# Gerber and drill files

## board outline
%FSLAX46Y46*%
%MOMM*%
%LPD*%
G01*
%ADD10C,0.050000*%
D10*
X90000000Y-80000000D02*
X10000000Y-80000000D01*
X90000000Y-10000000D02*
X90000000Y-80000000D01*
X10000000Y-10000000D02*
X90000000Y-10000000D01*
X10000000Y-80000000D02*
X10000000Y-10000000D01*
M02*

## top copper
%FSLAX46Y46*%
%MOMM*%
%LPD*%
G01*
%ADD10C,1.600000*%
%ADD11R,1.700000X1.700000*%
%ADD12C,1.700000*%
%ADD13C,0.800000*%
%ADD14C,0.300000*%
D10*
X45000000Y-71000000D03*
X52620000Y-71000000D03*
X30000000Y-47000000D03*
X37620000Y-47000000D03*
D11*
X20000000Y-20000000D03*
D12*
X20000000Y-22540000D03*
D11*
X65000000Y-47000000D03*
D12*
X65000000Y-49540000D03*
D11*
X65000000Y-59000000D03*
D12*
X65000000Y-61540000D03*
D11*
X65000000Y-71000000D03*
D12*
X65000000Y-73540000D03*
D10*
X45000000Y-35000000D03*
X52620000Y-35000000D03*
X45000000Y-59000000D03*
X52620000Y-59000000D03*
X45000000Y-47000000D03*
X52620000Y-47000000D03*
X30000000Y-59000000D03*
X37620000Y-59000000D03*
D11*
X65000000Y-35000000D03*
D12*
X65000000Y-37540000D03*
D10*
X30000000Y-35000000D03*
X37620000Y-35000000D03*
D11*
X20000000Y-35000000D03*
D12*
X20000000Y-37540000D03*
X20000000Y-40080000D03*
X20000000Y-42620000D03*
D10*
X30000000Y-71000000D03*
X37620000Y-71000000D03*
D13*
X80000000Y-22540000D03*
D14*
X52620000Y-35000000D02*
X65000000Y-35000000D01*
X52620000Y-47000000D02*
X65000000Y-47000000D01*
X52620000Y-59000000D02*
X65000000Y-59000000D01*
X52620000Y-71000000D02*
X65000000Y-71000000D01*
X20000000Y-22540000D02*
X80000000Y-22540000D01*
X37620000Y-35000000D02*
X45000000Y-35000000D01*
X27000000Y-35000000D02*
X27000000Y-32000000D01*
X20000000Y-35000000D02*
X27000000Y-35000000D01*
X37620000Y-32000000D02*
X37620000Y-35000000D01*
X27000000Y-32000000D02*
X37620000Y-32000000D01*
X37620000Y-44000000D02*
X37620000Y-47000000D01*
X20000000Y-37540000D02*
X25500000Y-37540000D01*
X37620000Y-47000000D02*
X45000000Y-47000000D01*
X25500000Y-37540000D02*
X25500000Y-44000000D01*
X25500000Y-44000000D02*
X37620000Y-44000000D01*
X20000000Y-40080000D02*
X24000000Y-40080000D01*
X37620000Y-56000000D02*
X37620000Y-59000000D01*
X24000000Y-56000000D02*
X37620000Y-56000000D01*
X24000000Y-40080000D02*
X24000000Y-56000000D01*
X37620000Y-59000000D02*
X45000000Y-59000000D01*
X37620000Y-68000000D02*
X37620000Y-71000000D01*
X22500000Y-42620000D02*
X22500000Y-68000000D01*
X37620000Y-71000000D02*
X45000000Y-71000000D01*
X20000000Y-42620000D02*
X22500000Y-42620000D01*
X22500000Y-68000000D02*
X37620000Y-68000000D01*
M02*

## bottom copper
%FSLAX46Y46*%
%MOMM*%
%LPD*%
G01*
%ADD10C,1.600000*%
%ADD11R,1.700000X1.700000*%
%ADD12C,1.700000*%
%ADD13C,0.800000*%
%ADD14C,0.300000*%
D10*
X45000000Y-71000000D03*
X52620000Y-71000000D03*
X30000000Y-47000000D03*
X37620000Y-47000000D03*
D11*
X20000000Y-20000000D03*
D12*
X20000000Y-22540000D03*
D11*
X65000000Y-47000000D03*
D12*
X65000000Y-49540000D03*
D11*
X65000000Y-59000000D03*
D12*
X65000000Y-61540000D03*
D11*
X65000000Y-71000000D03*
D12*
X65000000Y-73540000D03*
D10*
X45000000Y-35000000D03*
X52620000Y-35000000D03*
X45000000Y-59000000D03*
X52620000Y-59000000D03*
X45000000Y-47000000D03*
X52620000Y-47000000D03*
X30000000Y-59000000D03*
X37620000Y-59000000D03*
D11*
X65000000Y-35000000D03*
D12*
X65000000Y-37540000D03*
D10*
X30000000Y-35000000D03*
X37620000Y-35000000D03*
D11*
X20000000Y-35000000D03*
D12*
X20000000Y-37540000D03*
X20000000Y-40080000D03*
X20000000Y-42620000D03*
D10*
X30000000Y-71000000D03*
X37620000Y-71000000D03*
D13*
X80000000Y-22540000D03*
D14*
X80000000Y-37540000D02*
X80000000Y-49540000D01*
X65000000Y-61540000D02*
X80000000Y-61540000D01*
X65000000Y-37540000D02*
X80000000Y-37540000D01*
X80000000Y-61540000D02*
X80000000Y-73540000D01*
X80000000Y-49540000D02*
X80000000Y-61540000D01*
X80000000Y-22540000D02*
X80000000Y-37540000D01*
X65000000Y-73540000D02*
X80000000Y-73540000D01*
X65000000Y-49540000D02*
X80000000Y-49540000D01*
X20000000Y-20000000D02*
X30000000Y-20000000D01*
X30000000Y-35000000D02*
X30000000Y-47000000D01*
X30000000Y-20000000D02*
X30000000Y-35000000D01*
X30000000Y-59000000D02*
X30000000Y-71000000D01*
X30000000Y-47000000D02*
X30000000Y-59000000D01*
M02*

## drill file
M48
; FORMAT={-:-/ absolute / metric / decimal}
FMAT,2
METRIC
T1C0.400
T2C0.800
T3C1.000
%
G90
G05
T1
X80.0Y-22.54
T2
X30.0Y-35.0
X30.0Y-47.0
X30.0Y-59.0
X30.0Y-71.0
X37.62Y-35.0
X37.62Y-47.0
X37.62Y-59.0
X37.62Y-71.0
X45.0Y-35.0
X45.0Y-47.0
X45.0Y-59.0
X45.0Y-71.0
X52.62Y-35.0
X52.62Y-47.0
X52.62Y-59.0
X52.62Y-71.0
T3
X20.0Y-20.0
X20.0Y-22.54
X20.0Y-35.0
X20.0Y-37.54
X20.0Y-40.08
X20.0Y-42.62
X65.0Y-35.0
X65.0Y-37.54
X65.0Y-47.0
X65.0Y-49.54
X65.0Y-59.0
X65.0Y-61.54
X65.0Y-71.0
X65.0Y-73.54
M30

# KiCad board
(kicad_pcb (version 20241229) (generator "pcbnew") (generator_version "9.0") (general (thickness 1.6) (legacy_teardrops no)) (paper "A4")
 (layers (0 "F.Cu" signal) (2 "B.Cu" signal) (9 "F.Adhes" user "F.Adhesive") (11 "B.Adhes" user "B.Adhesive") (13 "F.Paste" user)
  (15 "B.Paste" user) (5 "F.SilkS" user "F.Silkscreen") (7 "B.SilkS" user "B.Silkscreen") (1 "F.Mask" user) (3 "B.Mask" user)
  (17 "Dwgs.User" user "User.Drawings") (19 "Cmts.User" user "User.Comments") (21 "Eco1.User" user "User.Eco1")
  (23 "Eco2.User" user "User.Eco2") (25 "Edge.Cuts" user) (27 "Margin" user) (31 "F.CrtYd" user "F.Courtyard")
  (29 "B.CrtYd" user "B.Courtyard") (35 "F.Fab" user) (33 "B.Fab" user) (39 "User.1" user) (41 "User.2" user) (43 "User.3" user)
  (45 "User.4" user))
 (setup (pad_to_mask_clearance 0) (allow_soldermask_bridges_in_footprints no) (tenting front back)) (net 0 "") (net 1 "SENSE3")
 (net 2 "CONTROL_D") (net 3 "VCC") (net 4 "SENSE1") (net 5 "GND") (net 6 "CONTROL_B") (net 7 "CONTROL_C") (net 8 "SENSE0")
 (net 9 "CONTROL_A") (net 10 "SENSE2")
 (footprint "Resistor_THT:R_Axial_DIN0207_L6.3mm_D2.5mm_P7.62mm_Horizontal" (layer "F.Cu") (at 45 71)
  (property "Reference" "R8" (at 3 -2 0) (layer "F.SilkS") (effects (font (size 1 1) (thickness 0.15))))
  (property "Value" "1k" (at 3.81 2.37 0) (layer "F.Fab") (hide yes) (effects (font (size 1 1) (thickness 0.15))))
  (pad "1" thru_hole circle (at 0 0) (size 1.6 1.6) (drill 0.8) (layers "*.Cu" "*.Mask") (remove_unused_layers no) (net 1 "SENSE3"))
  (pad "2" thru_hole circle (at 7.62 0) (size 1.6 1.6) (drill 0.8) (layers "*.Cu" "*.Mask") (remove_unused_layers no) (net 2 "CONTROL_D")))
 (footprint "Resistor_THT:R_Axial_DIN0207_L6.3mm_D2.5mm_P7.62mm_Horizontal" (layer "F.Cu") (at 30 47)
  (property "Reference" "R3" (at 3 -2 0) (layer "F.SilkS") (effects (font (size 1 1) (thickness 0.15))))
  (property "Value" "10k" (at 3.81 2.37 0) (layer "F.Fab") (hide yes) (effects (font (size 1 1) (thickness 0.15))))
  (pad "1" thru_hole circle (at 0 0) (size 1.6 1.6) (drill 0.8) (layers "*.Cu" "*.Mask") (remove_unused_layers no) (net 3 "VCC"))
  (pad "2" thru_hole circle (at 7.62 0) (size 1.6 1.6) (drill 0.8) (layers "*.Cu" "*.Mask") (remove_unused_layers no) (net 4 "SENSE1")))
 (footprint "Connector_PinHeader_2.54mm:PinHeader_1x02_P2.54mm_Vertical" (layer "F.Cu") (at 20 20)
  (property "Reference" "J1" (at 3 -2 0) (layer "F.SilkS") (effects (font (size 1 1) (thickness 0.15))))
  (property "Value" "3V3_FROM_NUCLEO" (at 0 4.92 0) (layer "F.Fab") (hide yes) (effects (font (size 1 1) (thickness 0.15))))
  (pad "1" thru_hole rect (at 0 0) (size 1.7 1.7) (drill 1) (layers "*.Cu" "*.Mask") (remove_unused_layers no) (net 3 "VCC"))
  (pad "2" thru_hole circle (at 0 2.54) (size 1.7 1.7) (drill 1) (layers "*.Cu" "*.Mask") (remove_unused_layers no) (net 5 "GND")))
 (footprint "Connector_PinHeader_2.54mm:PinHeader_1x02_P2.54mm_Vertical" (layer "F.Cu") (at 65 47)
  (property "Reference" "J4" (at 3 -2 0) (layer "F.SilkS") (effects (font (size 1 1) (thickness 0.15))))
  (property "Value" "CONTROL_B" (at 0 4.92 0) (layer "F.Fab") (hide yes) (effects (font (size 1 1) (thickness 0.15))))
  (pad "1" thru_hole rect (at 0 0) (size 1.7 1.7) (drill 1) (layers "*.Cu" "*.Mask") (remove_unused_layers no) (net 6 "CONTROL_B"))
  (pad "2" thru_hole circle (at 0 2.54) (size 1.7 1.7) (drill 1) (layers "*.Cu" "*.Mask") (remove_unused_layers no) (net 5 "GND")))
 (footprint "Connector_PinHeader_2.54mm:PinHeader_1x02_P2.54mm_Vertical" (layer "F.Cu") (at 65 59)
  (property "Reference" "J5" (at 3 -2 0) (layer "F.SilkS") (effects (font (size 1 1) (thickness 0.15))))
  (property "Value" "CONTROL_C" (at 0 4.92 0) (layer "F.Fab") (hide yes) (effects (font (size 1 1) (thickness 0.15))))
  (pad "1" thru_hole rect (at 0 0) (size 1.7 1.7) (drill 1) (layers "*.Cu" "*.Mask") (remove_unused_layers no) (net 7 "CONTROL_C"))
  (pad "2" thru_hole circle (at 0 2.54) (size 1.7 1.7) (drill 1) (layers "*.Cu" "*.Mask") (remove_unused_layers no) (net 5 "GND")))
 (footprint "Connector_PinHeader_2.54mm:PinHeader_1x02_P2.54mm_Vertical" (layer "F.Cu") (at 65 71)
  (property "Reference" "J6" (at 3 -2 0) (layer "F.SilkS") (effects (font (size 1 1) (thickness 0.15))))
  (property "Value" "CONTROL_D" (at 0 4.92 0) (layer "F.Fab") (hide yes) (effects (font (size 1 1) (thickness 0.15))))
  (pad "1" thru_hole rect (at 0 0) (size 1.7 1.7) (drill 1) (layers "*.Cu" "*.Mask") (remove_unused_layers no) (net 2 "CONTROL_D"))
  (pad "2" thru_hole circle (at 0 2.54) (size 1.7 1.7) (drill 1) (layers "*.Cu" "*.Mask") (remove_unused_layers no) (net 5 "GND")))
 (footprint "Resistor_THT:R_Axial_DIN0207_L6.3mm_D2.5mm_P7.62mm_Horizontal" (layer "F.Cu") (at 45 35)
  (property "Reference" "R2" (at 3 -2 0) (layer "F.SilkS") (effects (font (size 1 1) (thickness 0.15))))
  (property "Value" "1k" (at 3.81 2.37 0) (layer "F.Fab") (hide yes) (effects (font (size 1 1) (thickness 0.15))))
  (pad "1" thru_hole circle (at 0 0) (size 1.6 1.6) (drill 0.8) (layers "*.Cu" "*.Mask") (remove_unused_layers no) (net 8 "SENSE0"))
  (pad "2" thru_hole circle (at 7.62 0) (size 1.6 1.6) (drill 0.8) (layers "*.Cu" "*.Mask") (remove_unused_layers no) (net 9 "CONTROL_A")))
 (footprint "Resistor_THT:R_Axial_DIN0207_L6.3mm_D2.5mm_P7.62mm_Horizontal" (layer "F.Cu") (at 45 59)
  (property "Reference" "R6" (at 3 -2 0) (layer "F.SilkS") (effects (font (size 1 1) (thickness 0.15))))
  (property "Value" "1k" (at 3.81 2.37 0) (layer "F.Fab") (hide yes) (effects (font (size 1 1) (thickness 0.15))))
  (pad "1" thru_hole circle (at 0 0) (size 1.6 1.6) (drill 0.8) (layers "*.Cu" "*.Mask") (remove_unused_layers no) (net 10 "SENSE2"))
  (pad "2" thru_hole circle (at 7.62 0) (size 1.6 1.6) (drill 0.8) (layers "*.Cu" "*.Mask") (remove_unused_layers no) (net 7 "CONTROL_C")))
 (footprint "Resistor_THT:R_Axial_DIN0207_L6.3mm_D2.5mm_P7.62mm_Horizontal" (layer "F.Cu") (at 45 47)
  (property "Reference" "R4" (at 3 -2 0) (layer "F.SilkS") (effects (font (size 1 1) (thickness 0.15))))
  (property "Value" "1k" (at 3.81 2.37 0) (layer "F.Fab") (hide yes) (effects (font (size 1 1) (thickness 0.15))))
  (pad "1" thru_hole circle (at 0 0) (size 1.6 1.6) (drill 0.8) (layers "*.Cu" "*.Mask") (remove_unused_layers no) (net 4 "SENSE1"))
  (pad "2" thru_hole circle (at 7.62 0) (size 1.6 1.6) (drill 0.8) (layers "*.Cu" "*.Mask") (remove_unused_layers no) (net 6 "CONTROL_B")))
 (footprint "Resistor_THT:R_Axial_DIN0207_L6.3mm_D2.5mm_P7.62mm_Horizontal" (layer "F.Cu") (at 30 59)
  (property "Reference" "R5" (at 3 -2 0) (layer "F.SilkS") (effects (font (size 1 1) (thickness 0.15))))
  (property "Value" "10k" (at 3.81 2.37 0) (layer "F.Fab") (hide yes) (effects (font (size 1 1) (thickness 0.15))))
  (pad "1" thru_hole circle (at 0 0) (size 1.6 1.6) (drill 0.8) (layers "*.Cu" "*.Mask") (remove_unused_layers no) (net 3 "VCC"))
  (pad "2" thru_hole circle (at 7.62 0) (size 1.6 1.6) (drill 0.8) (layers "*.Cu" "*.Mask") (remove_unused_layers no) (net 10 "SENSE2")))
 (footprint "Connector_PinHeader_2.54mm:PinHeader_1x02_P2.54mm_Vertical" (layer "F.Cu") (at 65 35)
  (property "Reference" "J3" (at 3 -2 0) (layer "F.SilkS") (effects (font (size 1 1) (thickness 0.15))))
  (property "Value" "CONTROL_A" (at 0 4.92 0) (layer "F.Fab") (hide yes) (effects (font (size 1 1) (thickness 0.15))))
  (pad "1" thru_hole rect (at 0 0) (size 1.7 1.7) (drill 1) (layers "*.Cu" "*.Mask") (remove_unused_layers no) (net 9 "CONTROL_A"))
  (pad "2" thru_hole circle (at 0 2.54) (size 1.7 1.7) (drill 1) (layers "*.Cu" "*.Mask") (remove_unused_layers no) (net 5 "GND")))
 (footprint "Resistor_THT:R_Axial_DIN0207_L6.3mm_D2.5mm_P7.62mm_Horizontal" (layer "F.Cu") (at 30 35)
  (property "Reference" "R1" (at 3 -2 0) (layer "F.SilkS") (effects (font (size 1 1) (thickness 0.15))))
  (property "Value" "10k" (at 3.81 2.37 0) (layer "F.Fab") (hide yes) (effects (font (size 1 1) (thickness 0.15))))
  (pad "1" thru_hole circle (at 0 0) (size 1.6 1.6) (drill 0.8) (layers "*.Cu" "*.Mask") (remove_unused_layers no) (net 3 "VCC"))
  (pad "2" thru_hole circle (at 7.62 0) (size 1.6 1.6) (drill 0.8) (layers "*.Cu" "*.Mask") (remove_unused_layers no) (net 8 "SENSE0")))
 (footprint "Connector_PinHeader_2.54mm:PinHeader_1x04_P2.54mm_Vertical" (layer "F.Cu") (at 20 35)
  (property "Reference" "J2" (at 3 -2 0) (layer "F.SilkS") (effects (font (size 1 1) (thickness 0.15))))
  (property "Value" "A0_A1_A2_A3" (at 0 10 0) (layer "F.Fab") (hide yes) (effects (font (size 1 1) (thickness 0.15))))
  (pad "1" thru_hole rect (at 0 0) (size 1.7 1.7) (drill 1) (layers "*.Cu" "*.Mask") (remove_unused_layers no) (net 8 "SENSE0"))
  (pad "2" thru_hole circle (at 0 2.54) (size 1.7 1.7) (drill 1) (layers "*.Cu" "*.Mask") (remove_unused_layers no) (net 4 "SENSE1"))
  (pad "3" thru_hole circle (at 0 5.08) (size 1.7 1.7) (drill 1) (layers "*.Cu" "*.Mask") (remove_unused_layers no) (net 10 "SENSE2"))
  (pad "4" thru_hole circle (at 0 7.62) (size 1.7 1.7) (drill 1) (layers "*.Cu" "*.Mask") (remove_unused_layers no) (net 1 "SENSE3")))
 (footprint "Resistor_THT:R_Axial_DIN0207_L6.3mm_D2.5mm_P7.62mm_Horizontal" (layer "F.Cu") (at 30 71)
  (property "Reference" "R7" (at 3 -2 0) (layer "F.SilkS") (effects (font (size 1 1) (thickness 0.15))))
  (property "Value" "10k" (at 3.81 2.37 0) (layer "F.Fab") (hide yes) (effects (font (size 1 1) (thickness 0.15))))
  (pad "1" thru_hole circle (at 0 0) (size 1.6 1.6) (drill 0.8) (layers "*.Cu" "*.Mask") (remove_unused_layers no) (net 3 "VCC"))
  (pad "2" thru_hole circle (at 7.62 0) (size 1.6 1.6) (drill 0.8) (layers "*.Cu" "*.Mask") (remove_unused_layers no) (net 1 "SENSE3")))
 (gr_line (start 90 80) (end 10 80) (stroke (width 0.05) (type default)) (layer "Edge.Cuts"))
 (gr_line (start 90 10) (end 90 80) (stroke (width 0.05) (type default)) (layer "Edge.Cuts"))
 (gr_line (start 10 10) (end 90 10) (stroke (width 0.05) (type default)) (layer "Edge.Cuts"))
 (gr_line (start 10 80) (end 10 10) (stroke (width 0.05) (type default)) (layer "Edge.Cuts"))
 (segment (start 52.62 35) (end 65 35) (width 0.3) (layer "F.Cu") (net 9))
 (segment (start 52.62 47) (end 65 47) (width 0.3) (layer "F.Cu") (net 6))
 (segment (start 52.62 59) (end 65 59) (width 0.3) (layer "F.Cu") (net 7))
 (segment (start 52.62 71) (end 65 71) (width 0.3) (layer "F.Cu") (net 2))
 (segment (start 20 22.54) (end 80 22.54) (width 0.3) (layer "F.Cu") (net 5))
 (via (at 80 22.54) (size 0.8) (drill 0.4) (layers "F.Cu" "B.Cu") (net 5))
 (segment (start 80 37.54) (end 80 49.54) (width 0.3) (layer "B.Cu") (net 5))
 (segment (start 65 61.54) (end 80 61.54) (width 0.3) (layer "B.Cu") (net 5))
 (segment (start 65 37.54) (end 80 37.54) (width 0.3) (layer "B.Cu") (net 5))
 (segment (start 80 61.54) (end 80 73.54) (width 0.3) (layer "B.Cu") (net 5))
 (segment (start 80 49.54) (end 80 61.54) (width 0.3) (layer "B.Cu") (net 5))
 (segment (start 80 22.54) (end 80 37.54) (width 0.3) (layer "B.Cu") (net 5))
 (segment (start 65 73.54) (end 80 73.54) (width 0.3) (layer "B.Cu") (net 5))
 (segment (start 65 49.54) (end 80 49.54) (width 0.3) (layer "B.Cu") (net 5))
 (segment (start 37.62 35) (end 45 35) (width 0.3) (layer "F.Cu") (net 8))
 (segment (start 27 35) (end 27 32) (width 0.3) (layer "F.Cu") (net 8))
 (segment (start 20 35) (end 27 35) (width 0.3) (layer "F.Cu") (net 8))
 (segment (start 37.62 32) (end 37.62 35) (width 0.3) (layer "F.Cu") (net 8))
 (segment (start 27 32) (end 37.62 32) (width 0.3) (layer "F.Cu") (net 8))
 (segment (start 37.62 44) (end 37.62 47) (width 0.3) (layer "F.Cu") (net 4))
 (segment (start 20 37.54) (end 25.5 37.54) (width 0.3) (layer "F.Cu") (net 4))
 (segment (start 37.62 47) (end 45 47) (width 0.3) (layer "F.Cu") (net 4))
 (segment (start 25.5 37.54) (end 25.5 44) (width 0.3) (layer "F.Cu") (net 4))
 (segment (start 25.5 44) (end 37.62 44) (width 0.3) (layer "F.Cu") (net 4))
 (segment (start 20 40.08) (end 24 40.08) (width 0.3) (layer "F.Cu") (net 10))
 (segment (start 37.62 56) (end 37.62 59) (width 0.3) (layer "F.Cu") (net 10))
 (segment (start 24 56) (end 37.62 56) (width 0.3) (layer "F.Cu") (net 10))
 (segment (start 24 40.08) (end 24 56) (width 0.3) (layer "F.Cu") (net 10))
 (segment (start 37.62 59) (end 45 59) (width 0.3) (layer "F.Cu") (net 10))
 (segment (start 37.62 68) (end 37.62 71) (width 0.3) (layer "F.Cu") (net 1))
 (segment (start 22.5 42.62) (end 22.5 68) (width 0.3) (layer "F.Cu") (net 1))
 (segment (start 37.62 71) (end 45 71) (width 0.3) (layer "F.Cu") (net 1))
 (segment (start 20 42.62) (end 22.5 42.62) (width 0.3) (layer "F.Cu") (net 1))
 (segment (start 22.5 68) (end 37.62 68) (width 0.3) (layer "F.Cu") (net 1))
 (segment (start 20 20) (end 30 20) (width 0.3) (layer "B.Cu") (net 3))
 (segment (start 30 35) (end 30 47) (width 0.3) (layer "B.Cu") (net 3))
 (segment (start 30 20) (end 30 35) (width 0.3) (layer "B.Cu") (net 3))
 (segment (start 30 59) (end 30 71) (width 0.3) (layer "B.Cu") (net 3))
 (segment (start 30 47) (end 30 59) (width 0.3) (layer "B.Cu") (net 3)))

